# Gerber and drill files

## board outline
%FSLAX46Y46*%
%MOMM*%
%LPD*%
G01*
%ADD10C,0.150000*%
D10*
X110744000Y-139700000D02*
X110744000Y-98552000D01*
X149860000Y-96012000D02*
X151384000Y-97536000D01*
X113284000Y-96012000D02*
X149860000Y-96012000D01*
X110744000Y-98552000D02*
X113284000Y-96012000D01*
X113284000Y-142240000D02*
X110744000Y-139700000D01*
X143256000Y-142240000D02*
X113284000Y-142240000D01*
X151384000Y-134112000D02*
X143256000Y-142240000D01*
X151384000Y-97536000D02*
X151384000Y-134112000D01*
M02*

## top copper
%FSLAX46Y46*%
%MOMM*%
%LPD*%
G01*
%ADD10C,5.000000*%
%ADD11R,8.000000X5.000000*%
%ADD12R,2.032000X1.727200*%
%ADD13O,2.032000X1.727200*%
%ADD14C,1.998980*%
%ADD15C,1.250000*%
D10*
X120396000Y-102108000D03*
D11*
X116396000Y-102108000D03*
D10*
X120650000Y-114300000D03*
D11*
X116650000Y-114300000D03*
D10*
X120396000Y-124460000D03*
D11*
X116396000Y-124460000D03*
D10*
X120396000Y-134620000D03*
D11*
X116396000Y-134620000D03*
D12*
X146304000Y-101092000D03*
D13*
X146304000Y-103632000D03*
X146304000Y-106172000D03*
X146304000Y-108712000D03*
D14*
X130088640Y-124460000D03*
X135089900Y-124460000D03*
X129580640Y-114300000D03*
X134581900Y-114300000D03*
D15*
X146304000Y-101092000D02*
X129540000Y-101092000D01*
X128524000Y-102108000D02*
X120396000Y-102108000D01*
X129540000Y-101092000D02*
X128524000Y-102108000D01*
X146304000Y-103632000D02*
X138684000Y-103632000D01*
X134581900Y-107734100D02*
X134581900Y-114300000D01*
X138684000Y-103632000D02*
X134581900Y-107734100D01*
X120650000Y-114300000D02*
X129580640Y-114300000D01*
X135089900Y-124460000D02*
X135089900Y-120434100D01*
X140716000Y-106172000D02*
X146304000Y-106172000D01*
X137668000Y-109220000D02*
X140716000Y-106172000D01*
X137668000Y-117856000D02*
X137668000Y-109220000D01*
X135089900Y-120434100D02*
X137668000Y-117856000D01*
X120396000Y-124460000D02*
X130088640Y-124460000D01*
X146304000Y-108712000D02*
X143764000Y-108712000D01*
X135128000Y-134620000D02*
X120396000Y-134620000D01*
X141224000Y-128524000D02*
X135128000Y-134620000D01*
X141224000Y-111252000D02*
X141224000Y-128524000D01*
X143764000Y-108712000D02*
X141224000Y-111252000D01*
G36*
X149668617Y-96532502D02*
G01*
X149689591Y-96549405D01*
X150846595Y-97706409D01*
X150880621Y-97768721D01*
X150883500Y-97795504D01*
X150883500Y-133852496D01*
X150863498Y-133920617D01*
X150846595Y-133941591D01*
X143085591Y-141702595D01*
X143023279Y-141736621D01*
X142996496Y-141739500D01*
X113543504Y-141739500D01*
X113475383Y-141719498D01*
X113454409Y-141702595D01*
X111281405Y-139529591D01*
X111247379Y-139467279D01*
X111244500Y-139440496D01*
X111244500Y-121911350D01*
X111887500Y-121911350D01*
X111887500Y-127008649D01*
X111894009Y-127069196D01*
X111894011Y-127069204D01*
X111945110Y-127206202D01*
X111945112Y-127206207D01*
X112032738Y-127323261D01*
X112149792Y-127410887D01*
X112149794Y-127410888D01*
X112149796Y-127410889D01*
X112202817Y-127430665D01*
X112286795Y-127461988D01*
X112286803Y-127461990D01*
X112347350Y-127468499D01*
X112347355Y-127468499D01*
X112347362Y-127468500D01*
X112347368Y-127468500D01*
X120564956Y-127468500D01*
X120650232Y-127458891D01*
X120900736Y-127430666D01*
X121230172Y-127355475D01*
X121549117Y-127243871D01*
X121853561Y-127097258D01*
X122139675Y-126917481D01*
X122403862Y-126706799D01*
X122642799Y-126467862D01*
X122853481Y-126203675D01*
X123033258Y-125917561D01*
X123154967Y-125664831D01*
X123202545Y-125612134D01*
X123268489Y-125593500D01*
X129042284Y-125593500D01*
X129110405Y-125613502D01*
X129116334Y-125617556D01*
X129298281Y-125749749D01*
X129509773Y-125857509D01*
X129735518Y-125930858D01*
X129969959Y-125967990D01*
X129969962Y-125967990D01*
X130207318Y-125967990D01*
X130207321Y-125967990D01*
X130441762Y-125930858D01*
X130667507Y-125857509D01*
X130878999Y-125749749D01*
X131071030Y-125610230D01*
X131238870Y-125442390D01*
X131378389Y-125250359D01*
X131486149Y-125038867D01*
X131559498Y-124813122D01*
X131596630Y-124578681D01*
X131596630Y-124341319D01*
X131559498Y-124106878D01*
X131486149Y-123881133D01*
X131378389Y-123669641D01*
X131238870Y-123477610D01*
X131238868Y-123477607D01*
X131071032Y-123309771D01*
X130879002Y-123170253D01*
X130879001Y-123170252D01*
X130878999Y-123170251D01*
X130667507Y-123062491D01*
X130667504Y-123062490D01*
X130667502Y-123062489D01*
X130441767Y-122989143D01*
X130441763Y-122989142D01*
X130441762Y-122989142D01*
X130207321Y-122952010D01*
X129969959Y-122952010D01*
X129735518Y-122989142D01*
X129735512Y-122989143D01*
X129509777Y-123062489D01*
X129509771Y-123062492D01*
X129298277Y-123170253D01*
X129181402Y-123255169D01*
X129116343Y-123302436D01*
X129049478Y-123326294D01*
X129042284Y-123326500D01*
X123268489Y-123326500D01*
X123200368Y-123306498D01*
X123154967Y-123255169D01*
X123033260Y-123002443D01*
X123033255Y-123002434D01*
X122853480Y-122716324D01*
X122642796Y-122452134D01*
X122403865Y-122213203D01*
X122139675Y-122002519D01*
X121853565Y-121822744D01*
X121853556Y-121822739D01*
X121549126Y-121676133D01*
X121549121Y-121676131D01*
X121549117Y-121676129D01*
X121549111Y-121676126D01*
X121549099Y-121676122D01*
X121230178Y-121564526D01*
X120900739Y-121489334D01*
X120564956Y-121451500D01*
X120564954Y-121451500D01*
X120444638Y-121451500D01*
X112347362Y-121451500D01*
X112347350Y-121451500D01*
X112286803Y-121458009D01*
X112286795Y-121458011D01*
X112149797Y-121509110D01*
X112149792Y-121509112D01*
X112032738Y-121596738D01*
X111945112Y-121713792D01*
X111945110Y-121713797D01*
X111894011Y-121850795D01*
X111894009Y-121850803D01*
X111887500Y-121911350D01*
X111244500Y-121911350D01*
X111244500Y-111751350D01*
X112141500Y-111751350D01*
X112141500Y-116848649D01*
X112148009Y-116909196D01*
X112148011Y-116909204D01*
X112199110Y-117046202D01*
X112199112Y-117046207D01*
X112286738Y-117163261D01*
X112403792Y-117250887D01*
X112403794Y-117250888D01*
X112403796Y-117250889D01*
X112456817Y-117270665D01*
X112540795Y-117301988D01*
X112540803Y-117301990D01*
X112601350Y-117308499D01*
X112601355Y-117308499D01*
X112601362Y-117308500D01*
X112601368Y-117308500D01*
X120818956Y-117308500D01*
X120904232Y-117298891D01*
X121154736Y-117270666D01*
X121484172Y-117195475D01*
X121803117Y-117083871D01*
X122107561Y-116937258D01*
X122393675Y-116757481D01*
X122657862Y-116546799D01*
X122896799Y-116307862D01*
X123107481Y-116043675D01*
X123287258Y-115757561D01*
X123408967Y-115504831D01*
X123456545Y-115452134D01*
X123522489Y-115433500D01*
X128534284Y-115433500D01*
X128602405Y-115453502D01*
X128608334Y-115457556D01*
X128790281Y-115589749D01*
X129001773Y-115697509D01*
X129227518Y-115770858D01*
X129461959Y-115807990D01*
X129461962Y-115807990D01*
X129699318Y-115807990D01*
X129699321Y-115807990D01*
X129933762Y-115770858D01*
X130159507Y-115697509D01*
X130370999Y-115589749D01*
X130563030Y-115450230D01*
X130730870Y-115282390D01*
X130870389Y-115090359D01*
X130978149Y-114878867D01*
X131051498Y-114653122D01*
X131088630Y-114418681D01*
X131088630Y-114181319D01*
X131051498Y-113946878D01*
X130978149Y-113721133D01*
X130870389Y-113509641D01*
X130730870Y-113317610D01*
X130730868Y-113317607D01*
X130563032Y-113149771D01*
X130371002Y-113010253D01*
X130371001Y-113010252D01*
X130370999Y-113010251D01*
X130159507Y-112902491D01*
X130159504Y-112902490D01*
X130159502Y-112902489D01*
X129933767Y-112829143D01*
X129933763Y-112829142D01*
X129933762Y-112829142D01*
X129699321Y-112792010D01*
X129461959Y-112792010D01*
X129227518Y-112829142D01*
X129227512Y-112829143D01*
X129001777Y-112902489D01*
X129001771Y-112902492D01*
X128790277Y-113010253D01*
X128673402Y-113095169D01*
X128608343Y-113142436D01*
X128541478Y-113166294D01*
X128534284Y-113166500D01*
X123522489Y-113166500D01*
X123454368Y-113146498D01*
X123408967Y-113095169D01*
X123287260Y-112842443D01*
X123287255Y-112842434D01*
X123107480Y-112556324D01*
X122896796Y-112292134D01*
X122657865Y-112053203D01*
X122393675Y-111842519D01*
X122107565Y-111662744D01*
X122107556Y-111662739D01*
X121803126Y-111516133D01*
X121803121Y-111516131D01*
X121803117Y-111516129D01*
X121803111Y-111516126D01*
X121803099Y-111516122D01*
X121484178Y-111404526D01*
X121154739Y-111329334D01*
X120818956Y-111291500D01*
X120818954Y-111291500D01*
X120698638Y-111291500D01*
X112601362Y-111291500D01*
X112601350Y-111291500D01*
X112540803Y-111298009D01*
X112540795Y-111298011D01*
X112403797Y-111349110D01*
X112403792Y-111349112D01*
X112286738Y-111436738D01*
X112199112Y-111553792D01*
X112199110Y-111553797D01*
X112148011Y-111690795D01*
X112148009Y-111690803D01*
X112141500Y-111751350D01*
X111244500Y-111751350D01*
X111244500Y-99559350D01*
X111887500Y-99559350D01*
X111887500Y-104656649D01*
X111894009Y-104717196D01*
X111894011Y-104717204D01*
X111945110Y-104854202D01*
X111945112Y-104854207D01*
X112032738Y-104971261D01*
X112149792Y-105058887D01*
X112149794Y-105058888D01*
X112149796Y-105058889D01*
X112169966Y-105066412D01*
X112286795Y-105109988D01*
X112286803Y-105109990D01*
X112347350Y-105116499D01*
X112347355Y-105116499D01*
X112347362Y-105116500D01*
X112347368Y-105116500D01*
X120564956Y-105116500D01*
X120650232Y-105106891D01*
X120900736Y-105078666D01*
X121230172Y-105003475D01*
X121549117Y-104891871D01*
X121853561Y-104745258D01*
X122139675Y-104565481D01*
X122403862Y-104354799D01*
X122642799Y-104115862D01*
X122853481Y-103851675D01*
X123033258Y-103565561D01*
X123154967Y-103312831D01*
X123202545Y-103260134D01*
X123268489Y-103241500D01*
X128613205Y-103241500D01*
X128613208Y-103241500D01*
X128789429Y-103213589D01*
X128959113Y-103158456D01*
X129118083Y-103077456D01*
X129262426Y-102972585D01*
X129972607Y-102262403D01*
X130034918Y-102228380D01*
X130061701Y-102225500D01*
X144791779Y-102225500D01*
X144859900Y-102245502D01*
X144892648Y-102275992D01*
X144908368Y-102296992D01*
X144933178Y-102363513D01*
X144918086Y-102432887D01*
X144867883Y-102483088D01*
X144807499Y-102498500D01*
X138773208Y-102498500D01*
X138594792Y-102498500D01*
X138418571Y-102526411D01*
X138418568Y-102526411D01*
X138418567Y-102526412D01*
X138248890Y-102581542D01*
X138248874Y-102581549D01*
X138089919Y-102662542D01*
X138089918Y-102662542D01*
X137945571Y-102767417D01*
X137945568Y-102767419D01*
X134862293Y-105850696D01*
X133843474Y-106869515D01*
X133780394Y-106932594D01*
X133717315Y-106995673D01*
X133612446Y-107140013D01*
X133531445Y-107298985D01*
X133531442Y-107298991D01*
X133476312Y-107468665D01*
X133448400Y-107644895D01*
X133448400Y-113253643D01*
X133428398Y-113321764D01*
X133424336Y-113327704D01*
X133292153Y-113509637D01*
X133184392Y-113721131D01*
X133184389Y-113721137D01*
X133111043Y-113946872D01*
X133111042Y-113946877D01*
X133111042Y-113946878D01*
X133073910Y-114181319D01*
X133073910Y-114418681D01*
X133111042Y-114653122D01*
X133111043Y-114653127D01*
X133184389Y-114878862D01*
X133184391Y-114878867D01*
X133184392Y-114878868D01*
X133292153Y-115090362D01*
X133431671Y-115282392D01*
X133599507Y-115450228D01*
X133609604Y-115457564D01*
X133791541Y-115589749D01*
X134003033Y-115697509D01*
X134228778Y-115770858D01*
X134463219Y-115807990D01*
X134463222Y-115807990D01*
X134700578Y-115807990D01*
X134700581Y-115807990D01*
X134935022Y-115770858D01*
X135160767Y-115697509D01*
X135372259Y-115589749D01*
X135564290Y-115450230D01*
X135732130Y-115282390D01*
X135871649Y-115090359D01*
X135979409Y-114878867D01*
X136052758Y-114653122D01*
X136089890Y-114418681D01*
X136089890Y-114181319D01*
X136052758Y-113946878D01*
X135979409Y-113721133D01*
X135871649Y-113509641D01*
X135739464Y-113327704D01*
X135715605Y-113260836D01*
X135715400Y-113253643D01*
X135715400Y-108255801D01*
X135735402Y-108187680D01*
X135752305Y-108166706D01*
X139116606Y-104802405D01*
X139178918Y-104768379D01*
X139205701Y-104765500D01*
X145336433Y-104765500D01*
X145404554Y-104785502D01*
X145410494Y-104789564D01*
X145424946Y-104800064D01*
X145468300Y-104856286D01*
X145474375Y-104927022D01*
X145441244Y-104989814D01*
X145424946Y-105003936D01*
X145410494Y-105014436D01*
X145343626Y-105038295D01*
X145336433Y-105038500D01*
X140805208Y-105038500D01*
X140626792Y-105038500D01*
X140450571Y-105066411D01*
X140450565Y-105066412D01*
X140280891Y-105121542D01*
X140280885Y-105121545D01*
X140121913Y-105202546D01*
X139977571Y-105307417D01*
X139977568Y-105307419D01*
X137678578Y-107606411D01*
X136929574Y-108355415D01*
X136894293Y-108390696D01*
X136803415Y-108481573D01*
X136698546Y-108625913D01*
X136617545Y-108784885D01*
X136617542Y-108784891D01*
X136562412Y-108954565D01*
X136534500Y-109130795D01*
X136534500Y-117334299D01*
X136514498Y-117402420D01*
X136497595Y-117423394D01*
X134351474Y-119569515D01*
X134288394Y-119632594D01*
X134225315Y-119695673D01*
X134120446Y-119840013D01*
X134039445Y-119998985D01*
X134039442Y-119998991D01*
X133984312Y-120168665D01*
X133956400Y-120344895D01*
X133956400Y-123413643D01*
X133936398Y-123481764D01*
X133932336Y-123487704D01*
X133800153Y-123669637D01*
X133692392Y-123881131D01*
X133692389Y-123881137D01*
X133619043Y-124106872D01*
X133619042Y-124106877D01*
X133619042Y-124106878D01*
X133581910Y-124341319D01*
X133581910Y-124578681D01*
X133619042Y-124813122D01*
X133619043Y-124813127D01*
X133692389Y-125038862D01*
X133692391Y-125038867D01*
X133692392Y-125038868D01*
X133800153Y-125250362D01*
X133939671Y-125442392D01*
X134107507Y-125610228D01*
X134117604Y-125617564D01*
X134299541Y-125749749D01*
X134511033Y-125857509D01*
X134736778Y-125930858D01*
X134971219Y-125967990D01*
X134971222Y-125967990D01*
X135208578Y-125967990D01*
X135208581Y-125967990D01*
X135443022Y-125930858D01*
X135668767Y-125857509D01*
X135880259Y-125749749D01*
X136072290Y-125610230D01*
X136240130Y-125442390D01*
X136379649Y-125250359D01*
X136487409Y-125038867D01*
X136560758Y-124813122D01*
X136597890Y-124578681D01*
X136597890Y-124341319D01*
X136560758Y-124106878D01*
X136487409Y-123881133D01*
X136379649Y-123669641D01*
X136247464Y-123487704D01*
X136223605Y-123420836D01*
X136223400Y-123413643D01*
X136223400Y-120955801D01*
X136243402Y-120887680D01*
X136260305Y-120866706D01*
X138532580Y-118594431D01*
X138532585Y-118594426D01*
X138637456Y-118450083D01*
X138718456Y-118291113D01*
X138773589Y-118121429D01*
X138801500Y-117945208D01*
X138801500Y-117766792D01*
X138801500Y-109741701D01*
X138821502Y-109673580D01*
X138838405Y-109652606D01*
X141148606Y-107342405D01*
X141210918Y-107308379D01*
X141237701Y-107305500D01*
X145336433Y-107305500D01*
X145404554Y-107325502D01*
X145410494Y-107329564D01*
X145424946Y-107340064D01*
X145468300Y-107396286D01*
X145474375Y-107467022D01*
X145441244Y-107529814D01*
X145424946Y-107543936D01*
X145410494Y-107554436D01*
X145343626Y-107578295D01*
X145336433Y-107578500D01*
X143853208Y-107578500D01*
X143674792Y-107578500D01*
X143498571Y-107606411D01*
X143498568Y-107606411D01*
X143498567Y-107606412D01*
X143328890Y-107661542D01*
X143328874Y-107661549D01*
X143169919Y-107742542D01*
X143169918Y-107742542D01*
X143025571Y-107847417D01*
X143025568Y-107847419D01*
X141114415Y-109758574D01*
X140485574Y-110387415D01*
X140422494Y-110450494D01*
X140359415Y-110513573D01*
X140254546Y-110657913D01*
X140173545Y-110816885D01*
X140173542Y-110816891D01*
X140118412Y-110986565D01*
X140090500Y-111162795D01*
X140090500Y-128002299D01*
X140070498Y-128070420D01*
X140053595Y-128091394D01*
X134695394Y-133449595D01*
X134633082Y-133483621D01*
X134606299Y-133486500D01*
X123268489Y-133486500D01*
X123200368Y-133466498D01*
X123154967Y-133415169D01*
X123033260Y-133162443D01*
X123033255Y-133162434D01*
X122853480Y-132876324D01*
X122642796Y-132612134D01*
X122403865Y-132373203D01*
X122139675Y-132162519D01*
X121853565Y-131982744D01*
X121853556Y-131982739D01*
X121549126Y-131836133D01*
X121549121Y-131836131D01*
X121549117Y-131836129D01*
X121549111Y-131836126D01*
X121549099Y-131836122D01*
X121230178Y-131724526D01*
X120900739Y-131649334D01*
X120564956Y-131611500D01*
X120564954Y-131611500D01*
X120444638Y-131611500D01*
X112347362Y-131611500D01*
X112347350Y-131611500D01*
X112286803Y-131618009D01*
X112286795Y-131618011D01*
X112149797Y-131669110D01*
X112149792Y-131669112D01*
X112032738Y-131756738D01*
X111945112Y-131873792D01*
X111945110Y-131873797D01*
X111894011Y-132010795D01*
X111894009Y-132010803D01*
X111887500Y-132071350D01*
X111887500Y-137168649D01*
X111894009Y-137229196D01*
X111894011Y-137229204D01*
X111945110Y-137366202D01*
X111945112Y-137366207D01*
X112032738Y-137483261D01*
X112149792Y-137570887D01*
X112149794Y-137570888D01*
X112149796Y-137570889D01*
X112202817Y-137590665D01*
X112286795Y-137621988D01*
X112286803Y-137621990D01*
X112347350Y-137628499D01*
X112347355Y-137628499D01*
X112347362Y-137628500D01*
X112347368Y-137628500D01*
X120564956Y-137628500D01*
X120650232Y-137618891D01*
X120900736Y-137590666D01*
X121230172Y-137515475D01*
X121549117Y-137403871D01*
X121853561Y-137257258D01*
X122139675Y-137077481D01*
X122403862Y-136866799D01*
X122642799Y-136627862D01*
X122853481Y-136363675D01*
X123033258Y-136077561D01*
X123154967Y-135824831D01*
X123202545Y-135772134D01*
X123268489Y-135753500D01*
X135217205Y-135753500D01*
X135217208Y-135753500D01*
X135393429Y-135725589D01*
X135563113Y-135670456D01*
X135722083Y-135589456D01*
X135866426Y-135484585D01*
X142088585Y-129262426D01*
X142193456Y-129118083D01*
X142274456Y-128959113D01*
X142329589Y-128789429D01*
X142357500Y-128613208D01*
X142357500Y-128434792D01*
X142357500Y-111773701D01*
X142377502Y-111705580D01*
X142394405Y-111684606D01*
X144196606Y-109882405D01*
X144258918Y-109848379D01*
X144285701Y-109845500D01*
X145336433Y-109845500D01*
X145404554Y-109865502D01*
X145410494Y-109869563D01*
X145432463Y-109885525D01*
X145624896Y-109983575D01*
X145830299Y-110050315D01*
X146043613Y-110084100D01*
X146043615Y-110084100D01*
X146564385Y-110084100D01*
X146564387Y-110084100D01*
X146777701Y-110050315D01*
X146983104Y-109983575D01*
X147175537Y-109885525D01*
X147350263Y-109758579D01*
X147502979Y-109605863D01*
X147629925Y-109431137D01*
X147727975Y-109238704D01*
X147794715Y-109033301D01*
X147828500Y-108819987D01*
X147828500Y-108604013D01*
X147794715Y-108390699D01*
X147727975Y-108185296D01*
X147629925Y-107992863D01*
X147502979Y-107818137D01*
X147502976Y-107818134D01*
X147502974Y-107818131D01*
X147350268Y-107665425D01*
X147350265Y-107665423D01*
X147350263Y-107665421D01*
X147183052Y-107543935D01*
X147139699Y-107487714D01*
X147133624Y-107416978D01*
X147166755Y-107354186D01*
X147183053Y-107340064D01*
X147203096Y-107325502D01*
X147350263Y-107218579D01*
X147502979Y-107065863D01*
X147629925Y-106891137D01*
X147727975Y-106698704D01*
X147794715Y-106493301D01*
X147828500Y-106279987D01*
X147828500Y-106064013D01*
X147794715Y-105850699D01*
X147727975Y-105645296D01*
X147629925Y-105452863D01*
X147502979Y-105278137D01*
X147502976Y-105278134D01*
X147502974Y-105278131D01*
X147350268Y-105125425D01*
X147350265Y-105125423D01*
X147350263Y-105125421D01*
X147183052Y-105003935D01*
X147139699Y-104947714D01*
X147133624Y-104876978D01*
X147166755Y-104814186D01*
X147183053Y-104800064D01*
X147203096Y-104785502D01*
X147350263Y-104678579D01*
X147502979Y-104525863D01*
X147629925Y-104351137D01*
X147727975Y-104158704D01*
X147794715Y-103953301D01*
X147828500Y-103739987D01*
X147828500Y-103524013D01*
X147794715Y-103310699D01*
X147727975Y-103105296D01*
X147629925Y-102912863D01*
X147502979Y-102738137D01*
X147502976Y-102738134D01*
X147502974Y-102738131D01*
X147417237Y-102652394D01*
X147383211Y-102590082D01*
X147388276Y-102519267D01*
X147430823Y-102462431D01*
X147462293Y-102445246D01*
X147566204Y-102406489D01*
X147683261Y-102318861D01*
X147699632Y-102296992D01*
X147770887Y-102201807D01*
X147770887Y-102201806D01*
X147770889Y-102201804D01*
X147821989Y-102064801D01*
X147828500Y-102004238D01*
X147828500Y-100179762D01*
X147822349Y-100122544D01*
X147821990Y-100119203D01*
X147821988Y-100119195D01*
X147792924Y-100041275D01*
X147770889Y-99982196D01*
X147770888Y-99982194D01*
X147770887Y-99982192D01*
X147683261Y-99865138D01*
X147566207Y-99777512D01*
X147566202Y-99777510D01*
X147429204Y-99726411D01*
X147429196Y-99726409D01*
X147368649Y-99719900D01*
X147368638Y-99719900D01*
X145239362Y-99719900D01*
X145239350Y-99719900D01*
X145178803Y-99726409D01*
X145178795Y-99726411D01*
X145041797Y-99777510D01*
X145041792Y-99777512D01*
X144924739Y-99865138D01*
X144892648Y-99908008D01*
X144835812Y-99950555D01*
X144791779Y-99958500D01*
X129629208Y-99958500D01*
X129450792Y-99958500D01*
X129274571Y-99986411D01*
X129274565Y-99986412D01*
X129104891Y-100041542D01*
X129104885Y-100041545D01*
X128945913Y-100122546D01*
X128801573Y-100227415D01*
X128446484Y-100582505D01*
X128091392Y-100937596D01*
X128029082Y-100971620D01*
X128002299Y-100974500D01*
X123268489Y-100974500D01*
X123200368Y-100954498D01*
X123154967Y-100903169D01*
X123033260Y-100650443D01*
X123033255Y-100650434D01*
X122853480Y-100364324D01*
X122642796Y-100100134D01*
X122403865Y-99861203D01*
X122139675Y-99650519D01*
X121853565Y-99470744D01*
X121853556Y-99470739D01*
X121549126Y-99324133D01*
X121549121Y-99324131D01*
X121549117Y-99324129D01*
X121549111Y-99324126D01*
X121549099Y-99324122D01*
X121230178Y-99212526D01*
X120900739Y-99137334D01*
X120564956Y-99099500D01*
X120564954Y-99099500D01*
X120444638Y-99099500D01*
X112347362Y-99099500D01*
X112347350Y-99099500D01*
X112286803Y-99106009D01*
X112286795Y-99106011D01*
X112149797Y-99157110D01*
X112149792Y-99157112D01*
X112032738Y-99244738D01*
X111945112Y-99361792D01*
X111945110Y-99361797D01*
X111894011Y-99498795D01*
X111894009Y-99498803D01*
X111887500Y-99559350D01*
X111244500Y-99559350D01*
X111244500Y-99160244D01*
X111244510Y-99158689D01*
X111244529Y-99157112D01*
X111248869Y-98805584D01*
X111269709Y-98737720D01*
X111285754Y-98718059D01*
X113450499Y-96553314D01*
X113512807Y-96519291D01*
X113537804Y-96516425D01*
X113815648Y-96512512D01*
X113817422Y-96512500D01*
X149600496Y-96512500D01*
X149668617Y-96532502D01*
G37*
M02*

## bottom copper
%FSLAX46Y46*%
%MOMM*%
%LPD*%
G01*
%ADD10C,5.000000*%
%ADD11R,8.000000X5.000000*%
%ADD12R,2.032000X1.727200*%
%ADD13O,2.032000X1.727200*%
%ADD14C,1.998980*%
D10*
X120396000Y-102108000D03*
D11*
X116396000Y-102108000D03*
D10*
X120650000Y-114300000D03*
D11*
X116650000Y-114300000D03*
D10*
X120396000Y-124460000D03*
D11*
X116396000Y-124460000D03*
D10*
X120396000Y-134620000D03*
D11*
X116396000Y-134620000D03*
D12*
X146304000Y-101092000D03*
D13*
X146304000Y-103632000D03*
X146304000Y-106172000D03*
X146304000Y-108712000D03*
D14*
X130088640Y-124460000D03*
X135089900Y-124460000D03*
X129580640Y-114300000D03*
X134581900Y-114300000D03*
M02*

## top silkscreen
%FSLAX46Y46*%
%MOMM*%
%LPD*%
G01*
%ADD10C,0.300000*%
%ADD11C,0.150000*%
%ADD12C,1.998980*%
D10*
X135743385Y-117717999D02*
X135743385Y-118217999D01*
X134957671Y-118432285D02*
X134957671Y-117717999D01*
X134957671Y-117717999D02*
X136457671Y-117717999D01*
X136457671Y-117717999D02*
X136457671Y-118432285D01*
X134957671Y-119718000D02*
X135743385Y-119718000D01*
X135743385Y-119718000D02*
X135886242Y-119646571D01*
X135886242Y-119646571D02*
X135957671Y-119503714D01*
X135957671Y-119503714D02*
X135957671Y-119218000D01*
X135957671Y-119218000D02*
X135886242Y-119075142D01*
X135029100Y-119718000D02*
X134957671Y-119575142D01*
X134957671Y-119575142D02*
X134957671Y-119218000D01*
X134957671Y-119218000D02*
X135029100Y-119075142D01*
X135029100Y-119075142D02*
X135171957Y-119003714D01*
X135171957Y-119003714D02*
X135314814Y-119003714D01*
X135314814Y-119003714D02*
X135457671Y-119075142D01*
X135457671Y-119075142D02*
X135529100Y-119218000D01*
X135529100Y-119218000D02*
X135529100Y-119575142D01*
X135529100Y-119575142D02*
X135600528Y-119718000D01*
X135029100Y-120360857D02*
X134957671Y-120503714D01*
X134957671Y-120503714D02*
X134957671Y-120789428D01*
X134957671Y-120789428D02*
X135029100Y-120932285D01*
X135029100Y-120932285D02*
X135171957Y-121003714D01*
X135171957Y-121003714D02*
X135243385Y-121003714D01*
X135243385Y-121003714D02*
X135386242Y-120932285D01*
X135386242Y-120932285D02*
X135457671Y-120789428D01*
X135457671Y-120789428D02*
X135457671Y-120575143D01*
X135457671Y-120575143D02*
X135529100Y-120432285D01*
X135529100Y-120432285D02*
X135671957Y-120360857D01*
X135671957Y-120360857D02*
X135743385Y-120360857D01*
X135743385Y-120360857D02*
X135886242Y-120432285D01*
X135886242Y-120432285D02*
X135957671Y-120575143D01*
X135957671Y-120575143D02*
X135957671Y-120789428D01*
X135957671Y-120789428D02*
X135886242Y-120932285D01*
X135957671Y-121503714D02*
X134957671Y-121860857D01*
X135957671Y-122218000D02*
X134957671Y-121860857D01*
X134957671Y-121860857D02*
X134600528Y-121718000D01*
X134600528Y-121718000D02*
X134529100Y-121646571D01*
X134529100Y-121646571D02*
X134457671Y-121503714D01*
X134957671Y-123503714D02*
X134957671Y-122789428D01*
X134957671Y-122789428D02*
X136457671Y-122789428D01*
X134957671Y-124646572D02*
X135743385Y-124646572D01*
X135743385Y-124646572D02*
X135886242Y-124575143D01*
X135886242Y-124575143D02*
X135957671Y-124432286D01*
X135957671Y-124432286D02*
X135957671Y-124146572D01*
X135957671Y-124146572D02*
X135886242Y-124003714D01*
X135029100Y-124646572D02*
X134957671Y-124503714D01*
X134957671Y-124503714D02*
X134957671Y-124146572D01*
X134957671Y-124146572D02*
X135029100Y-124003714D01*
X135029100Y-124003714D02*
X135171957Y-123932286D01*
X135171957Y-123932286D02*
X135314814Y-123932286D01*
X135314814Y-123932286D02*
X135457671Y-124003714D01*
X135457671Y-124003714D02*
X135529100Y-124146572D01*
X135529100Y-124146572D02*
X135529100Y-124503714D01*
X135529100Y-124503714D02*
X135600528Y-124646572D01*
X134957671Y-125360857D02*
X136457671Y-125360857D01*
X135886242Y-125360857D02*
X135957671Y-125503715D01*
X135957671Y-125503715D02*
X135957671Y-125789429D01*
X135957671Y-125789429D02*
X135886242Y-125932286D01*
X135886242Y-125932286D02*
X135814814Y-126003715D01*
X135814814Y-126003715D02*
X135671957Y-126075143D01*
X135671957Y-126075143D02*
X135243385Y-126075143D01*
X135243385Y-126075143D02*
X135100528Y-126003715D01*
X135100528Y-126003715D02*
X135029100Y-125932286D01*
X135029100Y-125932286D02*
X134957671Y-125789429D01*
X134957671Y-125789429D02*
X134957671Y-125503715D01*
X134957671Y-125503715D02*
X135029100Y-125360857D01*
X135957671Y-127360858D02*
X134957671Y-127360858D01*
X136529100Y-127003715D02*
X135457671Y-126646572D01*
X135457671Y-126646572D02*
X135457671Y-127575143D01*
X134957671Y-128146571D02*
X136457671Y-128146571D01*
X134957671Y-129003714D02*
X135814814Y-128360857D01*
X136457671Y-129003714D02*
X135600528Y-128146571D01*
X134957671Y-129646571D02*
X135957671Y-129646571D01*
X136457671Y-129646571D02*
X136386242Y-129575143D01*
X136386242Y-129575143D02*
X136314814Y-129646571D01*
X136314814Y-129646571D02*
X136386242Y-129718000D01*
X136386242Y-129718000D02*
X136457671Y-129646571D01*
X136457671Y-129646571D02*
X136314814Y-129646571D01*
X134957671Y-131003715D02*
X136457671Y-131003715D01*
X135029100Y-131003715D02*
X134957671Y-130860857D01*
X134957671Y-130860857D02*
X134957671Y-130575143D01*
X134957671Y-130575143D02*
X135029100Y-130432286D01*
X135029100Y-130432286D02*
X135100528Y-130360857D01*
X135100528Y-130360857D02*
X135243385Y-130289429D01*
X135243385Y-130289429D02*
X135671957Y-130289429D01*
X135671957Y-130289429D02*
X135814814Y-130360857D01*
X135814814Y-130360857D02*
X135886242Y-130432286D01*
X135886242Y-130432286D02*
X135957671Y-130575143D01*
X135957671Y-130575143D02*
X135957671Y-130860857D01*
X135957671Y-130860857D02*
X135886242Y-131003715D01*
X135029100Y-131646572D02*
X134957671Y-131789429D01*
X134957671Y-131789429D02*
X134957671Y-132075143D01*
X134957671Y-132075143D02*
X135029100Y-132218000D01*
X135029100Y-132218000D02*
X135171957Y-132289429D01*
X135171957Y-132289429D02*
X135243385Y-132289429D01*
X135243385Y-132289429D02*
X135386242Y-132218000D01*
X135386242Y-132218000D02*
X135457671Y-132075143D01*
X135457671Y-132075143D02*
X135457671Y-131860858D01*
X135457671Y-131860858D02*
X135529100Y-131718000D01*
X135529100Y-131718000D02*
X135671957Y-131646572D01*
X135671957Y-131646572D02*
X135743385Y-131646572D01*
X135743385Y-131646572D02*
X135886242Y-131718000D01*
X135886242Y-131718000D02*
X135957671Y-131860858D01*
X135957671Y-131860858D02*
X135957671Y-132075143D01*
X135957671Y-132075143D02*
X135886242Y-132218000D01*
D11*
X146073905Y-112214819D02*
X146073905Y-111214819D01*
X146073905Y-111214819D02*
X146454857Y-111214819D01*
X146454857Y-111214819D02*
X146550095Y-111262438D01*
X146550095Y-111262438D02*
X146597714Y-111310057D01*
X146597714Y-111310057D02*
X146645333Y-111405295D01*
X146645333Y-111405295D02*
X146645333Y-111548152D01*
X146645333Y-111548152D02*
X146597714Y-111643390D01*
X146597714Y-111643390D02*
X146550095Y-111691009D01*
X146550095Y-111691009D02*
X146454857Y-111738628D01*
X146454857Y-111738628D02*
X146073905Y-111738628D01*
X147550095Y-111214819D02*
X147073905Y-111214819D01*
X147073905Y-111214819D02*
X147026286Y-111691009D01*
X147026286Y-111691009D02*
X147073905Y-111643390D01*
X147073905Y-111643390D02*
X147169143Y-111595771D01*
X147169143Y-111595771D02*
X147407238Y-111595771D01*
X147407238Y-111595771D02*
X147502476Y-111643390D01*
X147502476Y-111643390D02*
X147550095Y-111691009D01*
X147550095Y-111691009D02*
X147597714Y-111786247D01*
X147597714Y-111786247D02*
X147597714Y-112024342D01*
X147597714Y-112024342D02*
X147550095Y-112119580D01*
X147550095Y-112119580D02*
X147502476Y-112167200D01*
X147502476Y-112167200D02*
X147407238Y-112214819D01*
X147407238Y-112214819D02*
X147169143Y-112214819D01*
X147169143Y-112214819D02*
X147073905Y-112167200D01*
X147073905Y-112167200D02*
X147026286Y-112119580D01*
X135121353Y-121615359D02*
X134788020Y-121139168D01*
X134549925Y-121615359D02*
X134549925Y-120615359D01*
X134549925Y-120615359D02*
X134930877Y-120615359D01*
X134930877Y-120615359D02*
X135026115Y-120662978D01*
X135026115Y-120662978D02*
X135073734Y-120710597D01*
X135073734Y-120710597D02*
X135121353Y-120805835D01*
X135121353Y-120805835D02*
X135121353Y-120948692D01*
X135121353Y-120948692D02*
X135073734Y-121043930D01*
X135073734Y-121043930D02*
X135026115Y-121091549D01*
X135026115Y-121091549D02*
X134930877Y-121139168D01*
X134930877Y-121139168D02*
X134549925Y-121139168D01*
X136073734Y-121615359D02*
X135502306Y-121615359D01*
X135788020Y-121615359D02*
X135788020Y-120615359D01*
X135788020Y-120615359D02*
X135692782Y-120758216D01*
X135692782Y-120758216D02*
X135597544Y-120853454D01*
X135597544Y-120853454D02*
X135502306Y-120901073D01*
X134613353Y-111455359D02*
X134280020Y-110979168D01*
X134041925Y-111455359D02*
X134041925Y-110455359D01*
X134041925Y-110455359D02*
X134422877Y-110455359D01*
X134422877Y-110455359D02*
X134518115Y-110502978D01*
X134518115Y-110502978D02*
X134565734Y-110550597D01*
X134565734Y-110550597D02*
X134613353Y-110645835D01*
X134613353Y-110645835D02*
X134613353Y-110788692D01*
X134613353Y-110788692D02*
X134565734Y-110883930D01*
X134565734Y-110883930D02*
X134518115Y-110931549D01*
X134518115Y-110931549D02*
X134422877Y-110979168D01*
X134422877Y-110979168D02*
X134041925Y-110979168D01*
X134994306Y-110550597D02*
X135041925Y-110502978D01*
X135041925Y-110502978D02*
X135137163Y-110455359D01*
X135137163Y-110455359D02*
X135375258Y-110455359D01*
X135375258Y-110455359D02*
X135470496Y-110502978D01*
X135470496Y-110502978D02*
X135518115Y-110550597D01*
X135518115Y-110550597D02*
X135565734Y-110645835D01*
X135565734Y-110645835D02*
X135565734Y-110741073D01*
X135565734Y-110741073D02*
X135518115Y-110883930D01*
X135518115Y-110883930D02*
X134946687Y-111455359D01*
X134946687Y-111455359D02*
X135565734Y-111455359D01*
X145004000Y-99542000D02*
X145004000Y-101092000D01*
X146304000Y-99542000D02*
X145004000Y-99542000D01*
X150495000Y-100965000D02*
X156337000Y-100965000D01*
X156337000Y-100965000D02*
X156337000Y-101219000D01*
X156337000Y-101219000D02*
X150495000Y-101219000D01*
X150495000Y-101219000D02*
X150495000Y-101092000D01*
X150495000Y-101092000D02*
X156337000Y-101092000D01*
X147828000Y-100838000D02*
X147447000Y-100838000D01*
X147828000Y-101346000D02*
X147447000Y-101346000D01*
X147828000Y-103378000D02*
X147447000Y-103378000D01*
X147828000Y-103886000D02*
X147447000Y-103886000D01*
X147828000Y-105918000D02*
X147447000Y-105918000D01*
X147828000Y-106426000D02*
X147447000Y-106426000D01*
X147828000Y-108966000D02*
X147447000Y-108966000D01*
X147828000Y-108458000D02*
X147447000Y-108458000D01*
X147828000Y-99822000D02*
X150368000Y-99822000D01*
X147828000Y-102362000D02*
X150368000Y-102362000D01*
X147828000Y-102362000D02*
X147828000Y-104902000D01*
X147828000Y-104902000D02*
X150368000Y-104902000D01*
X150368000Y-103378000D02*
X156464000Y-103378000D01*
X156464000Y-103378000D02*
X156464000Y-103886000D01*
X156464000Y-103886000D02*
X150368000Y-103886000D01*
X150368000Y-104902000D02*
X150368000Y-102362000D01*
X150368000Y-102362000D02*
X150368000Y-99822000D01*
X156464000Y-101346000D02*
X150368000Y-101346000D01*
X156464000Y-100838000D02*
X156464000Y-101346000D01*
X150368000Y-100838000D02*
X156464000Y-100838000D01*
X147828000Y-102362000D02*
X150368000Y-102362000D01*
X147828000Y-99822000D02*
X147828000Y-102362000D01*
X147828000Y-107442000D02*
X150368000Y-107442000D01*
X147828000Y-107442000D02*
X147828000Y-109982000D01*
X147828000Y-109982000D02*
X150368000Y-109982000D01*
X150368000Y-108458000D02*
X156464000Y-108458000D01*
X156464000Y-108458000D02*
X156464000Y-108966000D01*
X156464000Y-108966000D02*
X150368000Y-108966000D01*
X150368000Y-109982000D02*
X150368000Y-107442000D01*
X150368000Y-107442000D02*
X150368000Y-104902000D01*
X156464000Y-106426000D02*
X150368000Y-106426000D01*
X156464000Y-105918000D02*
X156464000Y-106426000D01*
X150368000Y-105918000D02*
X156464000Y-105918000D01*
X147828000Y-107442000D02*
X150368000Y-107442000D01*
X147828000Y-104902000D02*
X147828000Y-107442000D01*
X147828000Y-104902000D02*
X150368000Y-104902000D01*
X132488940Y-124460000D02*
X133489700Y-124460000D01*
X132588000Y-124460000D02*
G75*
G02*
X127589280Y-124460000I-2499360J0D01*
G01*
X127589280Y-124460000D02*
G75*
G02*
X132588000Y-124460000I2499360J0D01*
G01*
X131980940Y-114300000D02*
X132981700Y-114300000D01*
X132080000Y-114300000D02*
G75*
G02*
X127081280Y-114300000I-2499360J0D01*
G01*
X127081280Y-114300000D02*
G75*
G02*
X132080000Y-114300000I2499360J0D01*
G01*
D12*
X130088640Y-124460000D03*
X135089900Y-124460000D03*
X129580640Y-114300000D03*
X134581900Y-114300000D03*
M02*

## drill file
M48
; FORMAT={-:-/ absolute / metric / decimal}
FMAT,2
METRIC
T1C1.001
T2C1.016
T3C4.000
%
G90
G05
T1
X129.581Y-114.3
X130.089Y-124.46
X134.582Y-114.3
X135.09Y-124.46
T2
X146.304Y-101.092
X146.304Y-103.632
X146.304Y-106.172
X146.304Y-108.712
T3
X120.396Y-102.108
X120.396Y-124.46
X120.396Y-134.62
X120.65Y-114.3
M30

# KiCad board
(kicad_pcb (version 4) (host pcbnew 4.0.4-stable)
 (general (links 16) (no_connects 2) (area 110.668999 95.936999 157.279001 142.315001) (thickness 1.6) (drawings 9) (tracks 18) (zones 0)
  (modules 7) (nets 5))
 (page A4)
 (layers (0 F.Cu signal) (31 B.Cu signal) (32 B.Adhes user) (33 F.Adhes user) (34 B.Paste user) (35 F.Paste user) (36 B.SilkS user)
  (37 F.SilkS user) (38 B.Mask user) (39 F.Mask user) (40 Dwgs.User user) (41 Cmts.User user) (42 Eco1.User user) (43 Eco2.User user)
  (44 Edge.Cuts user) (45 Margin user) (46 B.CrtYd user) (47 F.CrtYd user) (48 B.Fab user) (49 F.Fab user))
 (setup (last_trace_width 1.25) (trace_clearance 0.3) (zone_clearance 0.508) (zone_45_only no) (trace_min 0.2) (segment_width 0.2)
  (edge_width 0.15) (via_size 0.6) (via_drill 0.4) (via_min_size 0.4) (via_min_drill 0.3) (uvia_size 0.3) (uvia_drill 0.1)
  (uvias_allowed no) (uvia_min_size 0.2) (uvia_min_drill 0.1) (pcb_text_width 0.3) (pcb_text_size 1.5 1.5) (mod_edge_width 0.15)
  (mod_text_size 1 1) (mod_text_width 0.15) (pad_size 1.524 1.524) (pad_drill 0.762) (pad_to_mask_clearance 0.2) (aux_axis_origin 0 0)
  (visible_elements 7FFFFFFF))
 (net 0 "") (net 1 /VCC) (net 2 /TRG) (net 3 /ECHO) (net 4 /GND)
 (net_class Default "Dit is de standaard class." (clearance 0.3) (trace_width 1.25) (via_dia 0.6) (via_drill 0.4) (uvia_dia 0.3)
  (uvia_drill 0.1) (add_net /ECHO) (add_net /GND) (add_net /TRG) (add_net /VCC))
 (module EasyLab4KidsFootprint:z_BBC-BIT (layer F.Cu) (at 120.396 102.108 270)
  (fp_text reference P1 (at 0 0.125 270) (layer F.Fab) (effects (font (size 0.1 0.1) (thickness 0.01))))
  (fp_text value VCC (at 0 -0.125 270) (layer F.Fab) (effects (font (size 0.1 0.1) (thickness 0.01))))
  (pad 1 thru_hole circle (at 0 0 270) (size 5 5) (drill 4) (layers *.Cu *.Mask) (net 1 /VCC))
  (pad 1 smd rect (at 0 4 270) (size 5 8) (layers F.Cu F.Mask) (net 1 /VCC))
  (pad 1 smd rect (at 0 4 270) (size 5 8) (layers *.Mask B.Cu) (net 1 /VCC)))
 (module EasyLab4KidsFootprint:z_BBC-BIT (layer F.Cu) (at 120.65 114.3 270)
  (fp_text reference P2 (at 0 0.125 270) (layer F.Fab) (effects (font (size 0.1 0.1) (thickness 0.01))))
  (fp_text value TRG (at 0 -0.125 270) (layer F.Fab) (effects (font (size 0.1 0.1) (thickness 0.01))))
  (pad 1 thru_hole circle (at 0 0 270) (size 5 5) (drill 4) (layers *.Cu *.Mask) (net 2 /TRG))
  (pad 1 smd rect (at 0 4 270) (size 5 8) (layers F.Cu F.Mask) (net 2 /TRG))
  (pad 1 smd rect (at 0 4 270) (size 5 8) (layers *.Mask B.Cu) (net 2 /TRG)))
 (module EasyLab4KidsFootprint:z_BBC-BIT (layer F.Cu) (at 120.396 124.46 270)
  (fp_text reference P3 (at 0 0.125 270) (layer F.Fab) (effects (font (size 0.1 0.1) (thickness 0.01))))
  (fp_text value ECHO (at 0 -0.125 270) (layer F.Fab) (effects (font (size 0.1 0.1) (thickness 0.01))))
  (pad 1 thru_hole circle (at 0 0 270) (size 5 5) (drill 4) (layers *.Cu *.Mask) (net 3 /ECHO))
  (pad 1 smd rect (at 0 4 270) (size 5 8) (layers F.Cu F.Mask) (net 3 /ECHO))
  (pad 1 smd rect (at 0 4 270) (size 5 8) (layers *.Mask B.Cu) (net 3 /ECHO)))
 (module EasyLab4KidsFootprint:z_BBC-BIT (layer F.Cu) (at 120.396 134.62 270)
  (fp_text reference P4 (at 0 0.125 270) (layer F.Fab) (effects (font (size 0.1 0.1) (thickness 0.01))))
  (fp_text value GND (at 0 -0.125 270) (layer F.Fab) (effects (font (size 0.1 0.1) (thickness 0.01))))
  (pad 1 thru_hole circle (at 0 0 270) (size 5 5) (drill 4) (layers *.Cu *.Mask) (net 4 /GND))
  (pad 1 smd rect (at 0 4 270) (size 5 8) (layers F.Cu F.Mask) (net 4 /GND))
  (pad 1 smd rect (at 0 4 270) (size 5 8) (layers *.Mask B.Cu) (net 4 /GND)))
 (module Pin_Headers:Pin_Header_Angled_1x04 (layer F.Cu) (at 146.304 101.092)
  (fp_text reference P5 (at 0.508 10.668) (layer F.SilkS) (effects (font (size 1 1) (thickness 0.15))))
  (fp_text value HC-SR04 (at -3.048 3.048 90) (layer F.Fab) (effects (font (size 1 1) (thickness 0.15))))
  (fp_line (start -1.3 -1.55) (end -1.3 0) (layer F.SilkS) (width 0.15))
  (fp_line (start 0 -1.55) (end -1.3 -1.55) (layer F.SilkS) (width 0.15))
  (fp_line (start 4.191 -0.127) (end 10.033 -0.127) (layer F.SilkS) (width 0.15))
  (fp_line (start 10.033 -0.127) (end 10.033 0.127) (layer F.SilkS) (width 0.15))
  (fp_line (start 10.033 0.127) (end 4.191 0.127) (layer F.SilkS) (width 0.15))
  (fp_line (start 4.191 0.127) (end 4.191 0) (layer F.SilkS) (width 0.15))
  (fp_line (start 4.191 0) (end 10.033 0) (layer F.SilkS) (width 0.15))
  (fp_line (start 1.524 -0.254) (end 1.143 -0.254) (layer F.SilkS) (width 0.15))
  (fp_line (start 1.524 0.254) (end 1.143 0.254) (layer F.SilkS) (width 0.15))
  (fp_line (start 1.524 2.286) (end 1.143 2.286) (layer F.SilkS) (width 0.15))
  (fp_line (start 1.524 2.794) (end 1.143 2.794) (layer F.SilkS) (width 0.15))
  (fp_line (start 1.524 4.826) (end 1.143 4.826) (layer F.SilkS) (width 0.15))
  (fp_line (start 1.524 5.334) (end 1.143 5.334) (layer F.SilkS) (width 0.15))
  (fp_line (start 1.524 7.874) (end 1.143 7.874) (layer F.SilkS) (width 0.15))
  (fp_line (start 1.524 7.366) (end 1.143 7.366) (layer F.SilkS) (width 0.15))
  (fp_line (start 1.524 -1.27) (end 4.064 -1.27) (layer F.SilkS) (width 0.15))
  (fp_line (start 1.524 1.27) (end 4.064 1.27) (layer F.SilkS) (width 0.15))
  (fp_line (start 1.524 1.27) (end 1.524 3.81) (layer F.SilkS) (width 0.15))
  (fp_line (start 1.524 3.81) (end 4.064 3.81) (layer F.SilkS) (width 0.15))
  (fp_line (start 4.064 2.286) (end 10.16 2.286) (layer F.SilkS) (width 0.15))
  (fp_line (start 10.16 2.286) (end 10.16 2.794) (layer F.SilkS) (width 0.15))
  (fp_line (start 10.16 2.794) (end 4.064 2.794) (layer F.SilkS) (width 0.15))
  (fp_line (start 4.064 3.81) (end 4.064 1.27) (layer F.SilkS) (width 0.15))
  (fp_line (start 4.064 1.27) (end 4.064 -1.27) (layer F.SilkS) (width 0.15))
  (fp_line (start 10.16 0.254) (end 4.064 0.254) (layer F.SilkS) (width 0.15))
  (fp_line (start 10.16 -0.254) (end 10.16 0.254) (layer F.SilkS) (width 0.15))
  (fp_line (start 4.064 -0.254) (end 10.16 -0.254) (layer F.SilkS) (width 0.15))
  (fp_line (start 1.524 1.27) (end 4.064 1.27) (layer F.SilkS) (width 0.15))
  (fp_line (start 1.524 -1.27) (end 1.524 1.27) (layer F.SilkS) (width 0.15))
  (fp_line (start 1.524 6.35) (end 4.064 6.35) (layer F.SilkS) (width 0.15))
  (fp_line (start 1.524 6.35) (end 1.524 8.89) (layer F.SilkS) (width 0.15))
  (fp_line (start 1.524 8.89) (end 4.064 8.89) (layer F.SilkS) (width 0.15))
  (fp_line (start 4.064 7.366) (end 10.16 7.366) (layer F.SilkS) (width 0.15))
  (fp_line (start 10.16 7.366) (end 10.16 7.874) (layer F.SilkS) (width 0.15))
  (fp_line (start 10.16 7.874) (end 4.064 7.874) (layer F.SilkS) (width 0.15))
  (fp_line (start 4.064 8.89) (end 4.064 6.35) (layer F.SilkS) (width 0.15))
  (fp_line (start 4.064 6.35) (end 4.064 3.81) (layer F.SilkS) (width 0.15))
  (fp_line (start 10.16 5.334) (end 4.064 5.334) (layer F.SilkS) (width 0.15))
  (fp_line (start 10.16 4.826) (end 10.16 5.334) (layer F.SilkS) (width 0.15))
  (fp_line (start 4.064 4.826) (end 10.16 4.826) (layer F.SilkS) (width 0.15))
  (fp_line (start 1.524 6.35) (end 4.064 6.35) (layer F.SilkS) (width 0.15))
  (fp_line (start 1.524 3.81) (end 1.524 6.35) (layer F.SilkS) (width 0.15))
  (fp_line (start 1.524 3.81) (end 4.064 3.81) (layer F.SilkS) (width 0.15))
  (pad 1 thru_hole rect (at 0 0) (size 2.032 1.7272) (drill 1.016) (layers *.Cu *.Mask) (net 1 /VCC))
  (pad 2 thru_hole oval (at 0 2.54) (size 2.032 1.7272) (drill 1.016) (layers *.Cu *.Mask) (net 2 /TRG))
  (pad 3 thru_hole oval (at 0 5.08) (size 2.032 1.7272) (drill 1.016) (layers *.Cu *.Mask) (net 3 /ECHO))
  (pad 4 thru_hole oval (at 0 7.62) (size 2.032 1.7272) (drill 1.016) (layers *.Cu *.Mask) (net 4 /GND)))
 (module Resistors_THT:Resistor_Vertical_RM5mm (layer F.Cu) (at 132.588 124.46)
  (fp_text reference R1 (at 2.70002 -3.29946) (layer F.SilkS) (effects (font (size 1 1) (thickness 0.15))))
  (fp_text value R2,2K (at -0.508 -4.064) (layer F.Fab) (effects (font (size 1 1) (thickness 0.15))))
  (fp_line (start -0.09906 0) (end 0.9017 0) (layer F.SilkS) (width 0.15))
  (fp_circle (center -2.49936 0) (end 0 0) (layer F.SilkS) (width 0.15))
  (pad 1 thru_hole circle (at -2.49936 0) (size 1.99898 1.99898) (drill 1.00076) (layers *.Cu *.SilkS *.Mask) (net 3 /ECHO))
  (pad 2 thru_hole circle (at 2.5019 0) (size 1.99898 1.99898) (drill 1.00076) (layers *.Cu *.SilkS *.Mask) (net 3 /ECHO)))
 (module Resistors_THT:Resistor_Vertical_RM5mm (layer F.Cu) (at 132.08 114.3)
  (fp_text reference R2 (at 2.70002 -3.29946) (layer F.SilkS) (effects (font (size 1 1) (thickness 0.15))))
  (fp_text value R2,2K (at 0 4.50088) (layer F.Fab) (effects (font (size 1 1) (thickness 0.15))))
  (fp_line (start -0.09906 0) (end 0.9017 0) (layer F.SilkS) (width 0.15))
  (fp_circle (center -2.49936 0) (end 0 0) (layer F.SilkS) (width 0.15))
  (pad 1 thru_hole circle (at -2.49936 0) (size 1.99898 1.99898) (drill 1.00076) (layers *.Cu *.SilkS *.Mask) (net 2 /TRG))
  (pad 2 thru_hole circle (at 2.5019 0) (size 1.99898 1.99898) (drill 1.00076) (layers *.Cu *.SilkS *.Mask) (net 2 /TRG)))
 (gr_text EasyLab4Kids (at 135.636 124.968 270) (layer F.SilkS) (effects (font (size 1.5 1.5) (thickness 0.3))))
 (gr_line (start 110.744 139.7) (end 110.744 98.552) (angle 90) (layer Edge.Cuts) (width 0.15))
 (gr_line (start 149.86 96.012) (end 151.384 97.536) (angle 90) (layer Edge.Cuts) (width 0.15))
 (gr_line (start 113.284 96.012) (end 149.86 96.012) (angle 90) (layer Edge.Cuts) (width 0.15))
 (gr_line (start 110.744 98.552) (end 113.284 96.012) (angle 90) (layer Edge.Cuts) (width 0.15))
 (gr_line (start 113.284 142.24) (end 110.744 139.7) (angle 90) (layer Edge.Cuts) (width 0.15))
 (gr_line (start 143.256 142.24) (end 113.284 142.24) (angle 90) (layer Edge.Cuts) (width 0.15))
 (gr_line (start 151.384 134.112) (end 143.256 142.24) (angle 90) (layer Edge.Cuts) (width 0.15))
 (gr_line (start 151.384 97.536) (end 151.384 134.112) (angle 90) (layer Edge.Cuts) (width 0.15))
 (segment (start 146.304 101.092) (end 129.54 101.092) (width 1.25) (layer F.Cu) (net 1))
 (segment (start 128.524 102.108) (end 120.396 102.108) (width 1.25) (layer F.Cu) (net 1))
 (segment (start 129.54 101.092) (end 128.524 102.108) (width 1.25) (layer F.Cu) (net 1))
 (segment (start 146.304 103.632) (end 138.684 103.632) (width 1.25) (layer F.Cu) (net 2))
 (segment (start 134.5819 107.7341) (end 134.5819 114.3) (width 1.25) (layer F.Cu) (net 2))
 (segment (start 138.684 103.632) (end 134.5819 107.7341) (width 1.25) (layer F.Cu) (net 2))
 (segment (start 120.65 114.3) (end 129.58064 114.3) (width 1.25) (layer F.Cu) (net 2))
 (segment (start 135.0899 124.46) (end 135.0899 120.4341) (width 1.25) (layer F.Cu) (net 3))
 (segment (start 140.716 106.172) (end 146.304 106.172) (width 1.25) (layer F.Cu) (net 3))
 (segment (start 137.668 109.22) (end 140.716 106.172) (width 1.25) (layer F.Cu) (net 3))
 (segment (start 137.668 117.856) (end 137.668 109.22) (width 1.25) (layer F.Cu) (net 3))
 (segment (start 135.0899 120.4341) (end 137.668 117.856) (width 1.25) (layer F.Cu) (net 3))
 (segment (start 120.396 124.46) (end 130.08864 124.46) (width 1.25) (layer F.Cu) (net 3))
 (segment (start 146.304 108.712) (end 143.764 108.712) (width 1.25) (layer F.Cu) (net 4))
 (segment (start 135.128 134.62) (end 120.396 134.62) (width 1.25) (layer F.Cu) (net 4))
 (segment (start 141.224 128.524) (end 135.128 134.62) (width 1.25) (layer F.Cu) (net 4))
 (segment (start 141.224 111.252) (end 141.224 128.524) (width 1.25) (layer F.Cu) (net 4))
 (segment (start 143.764 108.712) (end 141.224 111.252) (width 1.25) (layer F.Cu) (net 4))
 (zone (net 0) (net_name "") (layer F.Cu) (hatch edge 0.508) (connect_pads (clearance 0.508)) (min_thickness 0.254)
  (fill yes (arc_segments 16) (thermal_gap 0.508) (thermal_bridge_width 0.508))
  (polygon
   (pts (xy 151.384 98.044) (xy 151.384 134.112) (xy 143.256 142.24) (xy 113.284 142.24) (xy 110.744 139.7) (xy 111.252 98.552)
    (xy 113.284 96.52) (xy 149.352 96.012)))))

